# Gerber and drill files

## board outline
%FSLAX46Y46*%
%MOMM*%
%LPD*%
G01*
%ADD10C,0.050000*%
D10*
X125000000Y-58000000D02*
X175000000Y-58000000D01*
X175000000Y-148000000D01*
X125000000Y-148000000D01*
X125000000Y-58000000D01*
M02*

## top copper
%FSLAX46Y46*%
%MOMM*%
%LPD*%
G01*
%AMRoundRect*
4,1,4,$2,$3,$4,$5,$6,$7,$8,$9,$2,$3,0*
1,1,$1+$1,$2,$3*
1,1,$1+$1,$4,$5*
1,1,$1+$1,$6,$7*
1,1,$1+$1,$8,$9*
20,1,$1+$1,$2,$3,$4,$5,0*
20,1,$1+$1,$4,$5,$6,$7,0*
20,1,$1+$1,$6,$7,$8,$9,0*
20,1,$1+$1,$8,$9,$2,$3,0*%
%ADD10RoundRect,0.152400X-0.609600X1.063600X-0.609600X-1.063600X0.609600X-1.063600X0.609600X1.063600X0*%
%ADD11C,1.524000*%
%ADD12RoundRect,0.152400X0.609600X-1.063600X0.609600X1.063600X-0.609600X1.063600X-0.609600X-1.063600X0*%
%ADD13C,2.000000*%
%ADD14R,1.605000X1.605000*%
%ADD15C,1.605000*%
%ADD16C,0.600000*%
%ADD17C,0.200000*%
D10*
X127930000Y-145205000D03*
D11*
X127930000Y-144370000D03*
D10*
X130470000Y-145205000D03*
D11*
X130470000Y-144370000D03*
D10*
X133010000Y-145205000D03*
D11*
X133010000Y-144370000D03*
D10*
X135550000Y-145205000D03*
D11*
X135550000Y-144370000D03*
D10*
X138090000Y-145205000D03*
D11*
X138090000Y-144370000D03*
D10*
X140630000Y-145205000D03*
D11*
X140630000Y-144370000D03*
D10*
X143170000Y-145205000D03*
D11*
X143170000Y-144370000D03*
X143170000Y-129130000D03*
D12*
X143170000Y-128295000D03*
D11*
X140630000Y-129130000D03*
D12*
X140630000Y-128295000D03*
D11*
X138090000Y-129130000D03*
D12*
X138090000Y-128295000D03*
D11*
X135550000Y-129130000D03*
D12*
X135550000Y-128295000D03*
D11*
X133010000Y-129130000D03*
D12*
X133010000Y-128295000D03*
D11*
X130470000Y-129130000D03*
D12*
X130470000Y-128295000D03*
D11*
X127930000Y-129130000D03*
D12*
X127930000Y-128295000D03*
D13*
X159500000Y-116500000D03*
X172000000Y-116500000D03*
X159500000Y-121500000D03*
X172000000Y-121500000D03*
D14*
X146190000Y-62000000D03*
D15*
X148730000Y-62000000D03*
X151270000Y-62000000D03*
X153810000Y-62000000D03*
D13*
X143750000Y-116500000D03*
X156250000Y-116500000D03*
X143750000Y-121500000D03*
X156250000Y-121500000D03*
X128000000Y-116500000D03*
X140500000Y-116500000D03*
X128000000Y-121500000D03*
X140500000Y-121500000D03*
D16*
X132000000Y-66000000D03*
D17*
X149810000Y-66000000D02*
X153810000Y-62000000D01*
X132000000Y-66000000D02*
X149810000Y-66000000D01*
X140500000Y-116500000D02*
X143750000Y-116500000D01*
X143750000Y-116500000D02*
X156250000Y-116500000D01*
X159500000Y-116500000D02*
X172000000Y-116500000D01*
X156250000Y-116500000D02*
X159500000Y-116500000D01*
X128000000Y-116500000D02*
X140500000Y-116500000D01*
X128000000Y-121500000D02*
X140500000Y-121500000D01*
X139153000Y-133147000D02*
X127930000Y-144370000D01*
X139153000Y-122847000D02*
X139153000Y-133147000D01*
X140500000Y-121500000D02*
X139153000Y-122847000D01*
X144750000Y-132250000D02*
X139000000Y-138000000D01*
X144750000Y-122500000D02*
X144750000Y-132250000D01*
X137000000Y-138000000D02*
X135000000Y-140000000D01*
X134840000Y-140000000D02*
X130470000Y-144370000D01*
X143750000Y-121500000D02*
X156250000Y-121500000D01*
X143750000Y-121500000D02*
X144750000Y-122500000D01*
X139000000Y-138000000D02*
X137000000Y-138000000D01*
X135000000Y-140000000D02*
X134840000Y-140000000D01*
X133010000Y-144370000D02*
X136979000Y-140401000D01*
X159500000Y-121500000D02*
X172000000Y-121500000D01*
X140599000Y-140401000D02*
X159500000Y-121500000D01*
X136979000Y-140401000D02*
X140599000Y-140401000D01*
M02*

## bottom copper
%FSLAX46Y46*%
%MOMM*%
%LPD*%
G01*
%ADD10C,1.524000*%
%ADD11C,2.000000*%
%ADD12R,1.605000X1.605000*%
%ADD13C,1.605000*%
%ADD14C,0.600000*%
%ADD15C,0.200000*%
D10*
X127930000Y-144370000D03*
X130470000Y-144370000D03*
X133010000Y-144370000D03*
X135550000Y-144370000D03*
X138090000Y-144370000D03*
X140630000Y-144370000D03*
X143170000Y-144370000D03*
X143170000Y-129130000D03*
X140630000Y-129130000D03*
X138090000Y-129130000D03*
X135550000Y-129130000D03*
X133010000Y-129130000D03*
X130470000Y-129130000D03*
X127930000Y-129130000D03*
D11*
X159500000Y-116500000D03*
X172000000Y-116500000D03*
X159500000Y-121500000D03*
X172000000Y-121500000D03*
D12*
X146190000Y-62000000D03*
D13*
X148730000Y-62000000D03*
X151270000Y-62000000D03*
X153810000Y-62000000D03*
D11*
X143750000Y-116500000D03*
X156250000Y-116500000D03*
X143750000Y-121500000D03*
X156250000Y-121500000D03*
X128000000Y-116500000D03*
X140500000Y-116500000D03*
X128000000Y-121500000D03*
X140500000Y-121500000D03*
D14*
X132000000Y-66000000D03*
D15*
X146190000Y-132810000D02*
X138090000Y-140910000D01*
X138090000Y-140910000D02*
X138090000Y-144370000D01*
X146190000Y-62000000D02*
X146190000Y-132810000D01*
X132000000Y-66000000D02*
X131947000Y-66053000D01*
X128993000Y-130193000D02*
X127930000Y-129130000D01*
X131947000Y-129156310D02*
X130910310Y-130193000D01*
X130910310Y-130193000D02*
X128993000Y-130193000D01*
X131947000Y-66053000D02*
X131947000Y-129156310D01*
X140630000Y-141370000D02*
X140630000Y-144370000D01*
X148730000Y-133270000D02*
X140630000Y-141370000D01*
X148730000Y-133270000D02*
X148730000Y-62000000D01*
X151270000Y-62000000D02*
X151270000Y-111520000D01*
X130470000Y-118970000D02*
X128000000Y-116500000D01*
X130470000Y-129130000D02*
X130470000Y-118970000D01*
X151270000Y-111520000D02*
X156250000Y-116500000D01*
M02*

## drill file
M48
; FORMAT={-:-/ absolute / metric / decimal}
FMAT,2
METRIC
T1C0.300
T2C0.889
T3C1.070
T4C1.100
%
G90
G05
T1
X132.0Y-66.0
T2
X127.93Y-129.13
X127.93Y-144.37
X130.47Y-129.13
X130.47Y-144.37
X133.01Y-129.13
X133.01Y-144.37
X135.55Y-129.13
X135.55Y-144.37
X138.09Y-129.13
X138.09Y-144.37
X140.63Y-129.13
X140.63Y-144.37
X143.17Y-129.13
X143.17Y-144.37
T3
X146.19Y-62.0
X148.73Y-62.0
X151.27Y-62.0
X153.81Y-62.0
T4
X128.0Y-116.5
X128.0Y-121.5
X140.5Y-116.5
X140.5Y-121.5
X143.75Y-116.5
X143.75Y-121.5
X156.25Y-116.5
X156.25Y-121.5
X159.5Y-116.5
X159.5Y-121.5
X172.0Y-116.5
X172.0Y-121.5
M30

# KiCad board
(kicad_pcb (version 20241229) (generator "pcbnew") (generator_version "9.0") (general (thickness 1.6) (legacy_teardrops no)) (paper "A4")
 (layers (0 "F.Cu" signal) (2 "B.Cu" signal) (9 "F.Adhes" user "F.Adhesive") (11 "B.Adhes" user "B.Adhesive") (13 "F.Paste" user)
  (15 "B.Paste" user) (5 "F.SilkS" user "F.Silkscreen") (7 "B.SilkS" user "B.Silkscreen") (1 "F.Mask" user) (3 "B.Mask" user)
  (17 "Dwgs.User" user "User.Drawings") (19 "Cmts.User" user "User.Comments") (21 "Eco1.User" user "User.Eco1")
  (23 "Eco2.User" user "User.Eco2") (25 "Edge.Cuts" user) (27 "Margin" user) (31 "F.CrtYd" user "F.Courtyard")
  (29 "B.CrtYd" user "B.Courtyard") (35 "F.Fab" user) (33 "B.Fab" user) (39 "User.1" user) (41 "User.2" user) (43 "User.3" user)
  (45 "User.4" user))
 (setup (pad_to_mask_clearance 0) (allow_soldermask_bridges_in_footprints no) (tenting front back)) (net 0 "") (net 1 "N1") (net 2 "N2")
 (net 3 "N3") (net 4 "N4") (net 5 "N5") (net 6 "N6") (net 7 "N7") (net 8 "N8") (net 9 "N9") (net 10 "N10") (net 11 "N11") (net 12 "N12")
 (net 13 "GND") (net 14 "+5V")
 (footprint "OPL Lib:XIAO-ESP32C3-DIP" (layer "F.Cu") (at 135.55 136.63 90)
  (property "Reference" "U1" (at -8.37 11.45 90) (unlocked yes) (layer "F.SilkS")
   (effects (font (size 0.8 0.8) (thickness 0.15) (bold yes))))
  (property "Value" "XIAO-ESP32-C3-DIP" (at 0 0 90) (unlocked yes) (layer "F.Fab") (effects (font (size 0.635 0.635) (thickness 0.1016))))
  (pad "1" smd roundrect (at -8.575 -7.62 270) (size 2.432 1.524) (layers "F.Cu" "F.Mask") (roundrect_rratio 0.1) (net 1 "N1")
   (thermal_bridge_angle 45))
  (pad "1" thru_hole circle (at -7.74 -7.62 270) (size 1.524 1.524) (drill 0.889) (layers "*.Cu" "*.Mask") (remove_unused_layers no)
   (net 1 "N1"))
  (pad "2" smd roundrect (at -8.575 -5.08 270) (size 2.432 1.524) (layers "F.Cu" "F.Mask") (roundrect_rratio 0.1) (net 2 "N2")
   (thermal_bridge_angle 45))
  (pad "2" thru_hole circle (at -7.74 -5.08 270) (size 1.524 1.524) (drill 0.889) (layers "*.Cu" "*.Mask") (remove_unused_layers no)
   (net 2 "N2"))
  (pad "3" smd roundrect (at -8.575 -2.54 270) (size 2.432 1.524) (layers "F.Cu" "F.Mask") (roundrect_rratio 0.1) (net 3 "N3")
   (thermal_bridge_angle 45))
  (pad "3" thru_hole circle (at -7.74 -2.54 270) (size 1.524 1.524) (drill 0.889) (layers "*.Cu" "*.Mask") (remove_unused_layers no)
   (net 3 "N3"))
  (pad "4" smd roundrect (at -8.575 0 270) (size 2.432 1.524) (layers "F.Cu" "F.Mask") (roundrect_rratio 0.1) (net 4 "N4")
   (thermal_bridge_angle 45))
  (pad "4" thru_hole circle (at -7.74 0 270) (size 1.524 1.524) (drill 0.889) (layers "*.Cu" "*.Mask") (remove_unused_layers no)
   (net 4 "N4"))
  (pad "5" smd roundrect (at -8.575 2.54 270) (size 2.432 1.524) (layers "F.Cu" "F.Mask") (roundrect_rratio 0.1) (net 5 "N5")
   (thermal_bridge_angle 45))
  (pad "5" thru_hole circle (at -7.74 2.54 270) (size 1.524 1.524) (drill 0.889) (layers "*.Cu" "*.Mask") (remove_unused_layers no)
   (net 5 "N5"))
  (pad "6" smd roundrect (at -8.575 5.08 270) (size 2.432 1.524) (layers "F.Cu" "F.Mask") (roundrect_rratio 0.1) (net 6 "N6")
   (thermal_bridge_angle 45))
  (pad "6" thru_hole circle (at -7.74 5.08 270) (size 1.524 1.524) (drill 0.889) (layers "*.Cu" "*.Mask") (remove_unused_layers no)
   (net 6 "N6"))
  (pad "7" smd roundrect (at -8.575 7.62 270) (size 2.432 1.524) (layers "F.Cu" "F.Mask") (roundrect_rratio 0.1) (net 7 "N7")
   (thermal_bridge_angle 45))
  (pad "7" thru_hole circle (at -7.74 7.62 270) (size 1.524 1.524) (drill 0.889) (layers "*.Cu" "*.Mask") (remove_unused_layers no)
   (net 7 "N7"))
  (pad "8" thru_hole circle (at 7.5 7.62 90) (size 1.524 1.524) (drill 0.889) (layers "*.Cu" "*.Mask") (remove_unused_layers no)
   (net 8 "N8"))
  (pad "8" smd roundrect (at 8.335 7.62 90) (size 2.432 1.524) (layers "F.Cu" "F.Mask") (roundrect_rratio 0.1) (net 8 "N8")
   (thermal_bridge_angle 45))
  (pad "9" thru_hole circle (at 7.5 5.08 90) (size 1.524 1.524) (drill 0.889) (layers "*.Cu" "*.Mask") (remove_unused_layers no)
   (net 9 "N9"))
  (pad "9" smd roundrect (at 8.335 5.08 90) (size 2.432 1.524) (layers "F.Cu" "F.Mask") (roundrect_rratio 0.1) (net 9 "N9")
   (thermal_bridge_angle 45))
  (pad "10" thru_hole circle (at 7.5 2.54 90) (size 1.524 1.524) (drill 0.889) (layers "*.Cu" "*.Mask") (remove_unused_layers no)
   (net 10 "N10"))
  (pad "10" smd roundrect (at 8.335 2.54 90) (size 2.432 1.524) (layers "F.Cu" "F.Mask") (roundrect_rratio 0.1) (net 10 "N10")
   (thermal_bridge_angle 45))
  (pad "11" thru_hole circle (at 7.5 0 90) (size 1.524 1.524) (drill 0.889) (layers "*.Cu" "*.Mask") (remove_unused_layers no)
   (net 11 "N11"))
  (pad "11" smd roundrect (at 8.335 0 90) (size 2.432 1.524) (layers "F.Cu" "F.Mask") (roundrect_rratio 0.1) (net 11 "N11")
   (thermal_bridge_angle 45))
  (pad "12" thru_hole circle (at 7.5 -2.54 90) (size 1.524 1.524) (drill 0.889) (layers "*.Cu" "*.Mask") (remove_unused_layers no)
   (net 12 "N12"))
  (pad "12" smd roundrect (at 8.335 -2.54 90) (size 2.432 1.524) (layers "F.Cu" "F.Mask") (roundrect_rratio 0.1) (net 12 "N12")
   (thermal_bridge_angle 45))
  (pad "13" thru_hole circle (at 7.5 -5.08 90) (size 1.524 1.524) (drill 0.889) (layers "*.Cu" "*.Mask") (remove_unused_layers no)
   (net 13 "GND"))
  (pad "13" smd roundrect (at 8.335 -5.08 90) (size 2.432 1.524) (layers "F.Cu" "F.Mask") (roundrect_rratio 0.1) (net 13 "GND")
   (thermal_bridge_angle 45))
  (pad "14" thru_hole circle (at 7.5 -7.62 90) (size 1.524 1.524) (drill 0.889) (layers "*.Cu" "*.Mask") (remove_unused_layers no)
   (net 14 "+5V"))
  (pad "14" smd roundrect (at 8.335 -7.62 90) (size 2.432 1.524) (layers "F.Cu" "F.Mask") (roundrect_rratio 0.1) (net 14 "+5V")
   (thermal_bridge_angle 45)))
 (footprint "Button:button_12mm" (layer "F.Cu") (at 165.75 119)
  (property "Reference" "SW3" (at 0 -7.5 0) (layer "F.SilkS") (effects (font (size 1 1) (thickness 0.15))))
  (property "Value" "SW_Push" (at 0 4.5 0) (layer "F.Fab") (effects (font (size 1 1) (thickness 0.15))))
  (pad "1" thru_hole circle (at -6.25 -2.5 90) (size 2 2) (drill 1.1) (layers "*.Cu" "*.Mask") (remove_unused_layers no) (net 13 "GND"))
  (pad "1" thru_hole circle (at 6.25 -2.5 90) (size 2 2) (drill 1.1) (layers "*.Cu" "*.Mask") (remove_unused_layers no) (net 13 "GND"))
  (pad "2" thru_hole circle (at -6.25 2.5 90) (size 2 2) (drill 1.1) (layers "*.Cu" "*.Mask") (remove_unused_layers no) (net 3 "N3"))
  (pad "2" thru_hole circle (at 6.25 2.5 90) (size 2 2) (drill 1.1) (layers "*.Cu" "*.Mask") (remove_unused_layers no) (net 3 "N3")))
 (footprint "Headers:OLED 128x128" (layer "F.Cu") (at 150 62)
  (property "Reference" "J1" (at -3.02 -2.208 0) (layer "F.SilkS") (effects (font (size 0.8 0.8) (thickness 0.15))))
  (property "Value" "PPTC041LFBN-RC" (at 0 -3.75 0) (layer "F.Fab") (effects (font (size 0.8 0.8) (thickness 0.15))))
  (pad "1" thru_hole rect (at -3.81 0) (size 1.605 1.605) (drill 1.07) (layers "*.Cu" "*.Mask") (remove_unused_layers no) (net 5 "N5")
   (solder_mask_margin 0.102))
  (pad "2" thru_hole circle (at -1.27 0) (size 1.605 1.605) (drill 1.07) (layers "*.Cu" "*.Mask") (remove_unused_layers no) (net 6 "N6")
   (solder_mask_margin 0.102))
  (pad "3" thru_hole circle (at 1.27 0) (size 1.605 1.605) (drill 1.07) (layers "*.Cu" "*.Mask") (remove_unused_layers no) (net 13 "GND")
   (solder_mask_margin 0.102))
  (pad "4" thru_hole circle (at 3.81 0) (size 1.605 1.605) (drill 1.07) (layers "*.Cu" "*.Mask") (remove_unused_layers no) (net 14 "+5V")
   (solder_mask_margin 0.102)))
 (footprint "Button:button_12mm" (layer "F.Cu") (at 150 119)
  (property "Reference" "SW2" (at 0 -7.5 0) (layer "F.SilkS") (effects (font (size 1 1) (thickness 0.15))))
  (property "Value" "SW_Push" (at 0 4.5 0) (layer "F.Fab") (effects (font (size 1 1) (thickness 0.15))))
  (pad "1" thru_hole circle (at -6.25 -2.5 90) (size 2 2) (drill 1.1) (layers "*.Cu" "*.Mask") (remove_unused_layers no) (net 13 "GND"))
  (pad "1" thru_hole circle (at 6.25 -2.5 90) (size 2 2) (drill 1.1) (layers "*.Cu" "*.Mask") (remove_unused_layers no) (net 13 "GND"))
  (pad "2" thru_hole circle (at -6.25 2.5 90) (size 2 2) (drill 1.1) (layers "*.Cu" "*.Mask") (remove_unused_layers no) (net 2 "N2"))
  (pad "2" thru_hole circle (at 6.25 2.5 90) (size 2 2) (drill 1.1) (layers "*.Cu" "*.Mask") (remove_unused_layers no) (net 2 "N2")))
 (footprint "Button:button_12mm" (layer "F.Cu") (at 134.25 119)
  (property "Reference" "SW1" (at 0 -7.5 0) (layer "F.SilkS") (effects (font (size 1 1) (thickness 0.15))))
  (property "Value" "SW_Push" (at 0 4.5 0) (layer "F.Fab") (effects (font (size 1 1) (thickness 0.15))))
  (pad "1" thru_hole circle (at -6.25 -2.5 90) (size 2 2) (drill 1.1) (layers "*.Cu" "*.Mask") (remove_unused_layers no) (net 13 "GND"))
  (pad "1" thru_hole circle (at 6.25 -2.5 90) (size 2 2) (drill 1.1) (layers "*.Cu" "*.Mask") (remove_unused_layers no) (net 13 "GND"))
  (pad "2" thru_hole circle (at -6.25 2.5 90) (size 2 2) (drill 1.1) (layers "*.Cu" "*.Mask") (remove_unused_layers no) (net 1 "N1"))
  (pad "2" thru_hole circle (at 6.25 2.5 90) (size 2 2) (drill 1.1) (layers "*.Cu" "*.Mask") (remove_unused_layers no) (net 1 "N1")))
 (gr_rect (start 125 58) (end 175 148) (stroke (width 0.05) (type solid)) (fill no) (layer "Edge.Cuts"))
 (segment (start 146.19 132.81) (end 138.09 140.91) (width 0.2) (layer "B.Cu") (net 5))
 (segment (start 138.09 140.91) (end 138.09 144.37) (width 0.2) (layer "B.Cu") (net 5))
 (segment (start 146.19 62) (end 146.19 132.81) (width 0.2) (layer "B.Cu") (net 5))
 (segment (start 149.81 66) (end 153.81 62) (width 0.2) (layer "F.Cu") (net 14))
 (segment (start 132 66) (end 149.81 66) (width 0.2) (layer "F.Cu") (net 14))
 (via (at 132 66) (size 0.6) (drill 0.3) (layers "F.Cu" "B.Cu") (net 14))
 (segment (start 132 66) (end 131.947 66.053) (width 0.2) (layer "B.Cu") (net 14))
 (segment (start 128.993 130.193) (end 127.93 129.13) (width 0.2) (layer "B.Cu") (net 14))
 (segment (start 131.947 129.15631) (end 130.91031 130.193) (width 0.2) (layer "B.Cu") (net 14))
 (segment (start 130.91031 130.193) (end 128.993 130.193) (width 0.2) (layer "B.Cu") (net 14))
 (segment (start 131.947 66.053) (end 131.947 129.15631) (width 0.2) (layer "B.Cu") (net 14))
 (segment (start 140.63 141.37) (end 140.63 144.37) (width 0.2) (layer "B.Cu") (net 6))
 (segment (start 148.73 133.27) (end 140.63 141.37) (width 0.2) (layer "B.Cu") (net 6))
 (segment (start 148.73 133.27) (end 148.73 62) (width 0.2) (layer "B.Cu") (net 6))
 (segment (start 140.5 116.5) (end 143.75 116.5) (width 0.2) (layer "F.Cu") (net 13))
 (segment (start 143.75 116.5) (end 156.25 116.5) (width 0.2) (layer "F.Cu") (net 13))
 (segment (start 159.5 116.5) (end 172 116.5) (width 0.2) (layer "F.Cu") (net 13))
 (segment (start 156.25 116.5) (end 159.5 116.5) (width 0.2) (layer "F.Cu") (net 13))
 (segment (start 128 116.5) (end 140.5 116.5) (width 0.2) (layer "F.Cu") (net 13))
 (segment (start 151.27 62) (end 151.27 111.52) (width 0.2) (layer "B.Cu") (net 13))
 (segment (start 130.47 118.97) (end 128 116.5) (width 0.2) (layer "B.Cu") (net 13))
 (segment (start 130.47 129.13) (end 130.47 118.97) (width 0.2) (layer "B.Cu") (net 13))
 (segment (start 151.27 111.52) (end 156.25 116.5) (width 0.2) (layer "B.Cu") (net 13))
 (segment (start 128 121.5) (end 140.5 121.5) (width 0.2) (layer "F.Cu") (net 1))
 (segment (start 139.153 133.147) (end 127.93 144.37) (width 0.2) (layer "F.Cu") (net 1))
 (segment (start 139.153 122.847) (end 139.153 133.147) (width 0.2) (layer "F.Cu") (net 1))
 (segment (start 140.5 121.5) (end 139.153 122.847) (width 0.2) (layer "F.Cu") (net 1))
 (segment (start 144.75 132.25) (end 139 138) (width 0.2) (layer "F.Cu") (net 2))
 (segment (start 144.75 122.5) (end 144.75 132.25) (width 0.2) (layer "F.Cu") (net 2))
 (segment (start 137 138) (end 135 140) (width 0.2) (layer "F.Cu") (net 2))
 (segment (start 134.84 140) (end 130.47 144.37) (width 0.2) (layer "F.Cu") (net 2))
 (segment (start 143.75 121.5) (end 156.25 121.5) (width 0.2) (layer "F.Cu") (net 2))
 (segment (start 143.75 121.5) (end 144.75 122.5) (width 0.2) (layer "F.Cu") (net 2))
 (segment (start 139 138) (end 137 138) (width 0.2) (layer "F.Cu") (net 2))
 (segment (start 135 140) (end 134.84 140) (width 0.2) (layer "F.Cu") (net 2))
 (segment (start 133.01 144.37) (end 136.979 140.401) (width 0.2) (layer "F.Cu") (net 3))
 (segment (start 159.5 121.5) (end 172 121.5) (width 0.2) (layer "F.Cu") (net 3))
 (segment (start 140.599 140.401) (end 159.5 121.5) (width 0.2) (layer "F.Cu") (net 3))
 (segment (start 136.979 140.401) (end 140.599 140.401) (width 0.2) (layer "F.Cu") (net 3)))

